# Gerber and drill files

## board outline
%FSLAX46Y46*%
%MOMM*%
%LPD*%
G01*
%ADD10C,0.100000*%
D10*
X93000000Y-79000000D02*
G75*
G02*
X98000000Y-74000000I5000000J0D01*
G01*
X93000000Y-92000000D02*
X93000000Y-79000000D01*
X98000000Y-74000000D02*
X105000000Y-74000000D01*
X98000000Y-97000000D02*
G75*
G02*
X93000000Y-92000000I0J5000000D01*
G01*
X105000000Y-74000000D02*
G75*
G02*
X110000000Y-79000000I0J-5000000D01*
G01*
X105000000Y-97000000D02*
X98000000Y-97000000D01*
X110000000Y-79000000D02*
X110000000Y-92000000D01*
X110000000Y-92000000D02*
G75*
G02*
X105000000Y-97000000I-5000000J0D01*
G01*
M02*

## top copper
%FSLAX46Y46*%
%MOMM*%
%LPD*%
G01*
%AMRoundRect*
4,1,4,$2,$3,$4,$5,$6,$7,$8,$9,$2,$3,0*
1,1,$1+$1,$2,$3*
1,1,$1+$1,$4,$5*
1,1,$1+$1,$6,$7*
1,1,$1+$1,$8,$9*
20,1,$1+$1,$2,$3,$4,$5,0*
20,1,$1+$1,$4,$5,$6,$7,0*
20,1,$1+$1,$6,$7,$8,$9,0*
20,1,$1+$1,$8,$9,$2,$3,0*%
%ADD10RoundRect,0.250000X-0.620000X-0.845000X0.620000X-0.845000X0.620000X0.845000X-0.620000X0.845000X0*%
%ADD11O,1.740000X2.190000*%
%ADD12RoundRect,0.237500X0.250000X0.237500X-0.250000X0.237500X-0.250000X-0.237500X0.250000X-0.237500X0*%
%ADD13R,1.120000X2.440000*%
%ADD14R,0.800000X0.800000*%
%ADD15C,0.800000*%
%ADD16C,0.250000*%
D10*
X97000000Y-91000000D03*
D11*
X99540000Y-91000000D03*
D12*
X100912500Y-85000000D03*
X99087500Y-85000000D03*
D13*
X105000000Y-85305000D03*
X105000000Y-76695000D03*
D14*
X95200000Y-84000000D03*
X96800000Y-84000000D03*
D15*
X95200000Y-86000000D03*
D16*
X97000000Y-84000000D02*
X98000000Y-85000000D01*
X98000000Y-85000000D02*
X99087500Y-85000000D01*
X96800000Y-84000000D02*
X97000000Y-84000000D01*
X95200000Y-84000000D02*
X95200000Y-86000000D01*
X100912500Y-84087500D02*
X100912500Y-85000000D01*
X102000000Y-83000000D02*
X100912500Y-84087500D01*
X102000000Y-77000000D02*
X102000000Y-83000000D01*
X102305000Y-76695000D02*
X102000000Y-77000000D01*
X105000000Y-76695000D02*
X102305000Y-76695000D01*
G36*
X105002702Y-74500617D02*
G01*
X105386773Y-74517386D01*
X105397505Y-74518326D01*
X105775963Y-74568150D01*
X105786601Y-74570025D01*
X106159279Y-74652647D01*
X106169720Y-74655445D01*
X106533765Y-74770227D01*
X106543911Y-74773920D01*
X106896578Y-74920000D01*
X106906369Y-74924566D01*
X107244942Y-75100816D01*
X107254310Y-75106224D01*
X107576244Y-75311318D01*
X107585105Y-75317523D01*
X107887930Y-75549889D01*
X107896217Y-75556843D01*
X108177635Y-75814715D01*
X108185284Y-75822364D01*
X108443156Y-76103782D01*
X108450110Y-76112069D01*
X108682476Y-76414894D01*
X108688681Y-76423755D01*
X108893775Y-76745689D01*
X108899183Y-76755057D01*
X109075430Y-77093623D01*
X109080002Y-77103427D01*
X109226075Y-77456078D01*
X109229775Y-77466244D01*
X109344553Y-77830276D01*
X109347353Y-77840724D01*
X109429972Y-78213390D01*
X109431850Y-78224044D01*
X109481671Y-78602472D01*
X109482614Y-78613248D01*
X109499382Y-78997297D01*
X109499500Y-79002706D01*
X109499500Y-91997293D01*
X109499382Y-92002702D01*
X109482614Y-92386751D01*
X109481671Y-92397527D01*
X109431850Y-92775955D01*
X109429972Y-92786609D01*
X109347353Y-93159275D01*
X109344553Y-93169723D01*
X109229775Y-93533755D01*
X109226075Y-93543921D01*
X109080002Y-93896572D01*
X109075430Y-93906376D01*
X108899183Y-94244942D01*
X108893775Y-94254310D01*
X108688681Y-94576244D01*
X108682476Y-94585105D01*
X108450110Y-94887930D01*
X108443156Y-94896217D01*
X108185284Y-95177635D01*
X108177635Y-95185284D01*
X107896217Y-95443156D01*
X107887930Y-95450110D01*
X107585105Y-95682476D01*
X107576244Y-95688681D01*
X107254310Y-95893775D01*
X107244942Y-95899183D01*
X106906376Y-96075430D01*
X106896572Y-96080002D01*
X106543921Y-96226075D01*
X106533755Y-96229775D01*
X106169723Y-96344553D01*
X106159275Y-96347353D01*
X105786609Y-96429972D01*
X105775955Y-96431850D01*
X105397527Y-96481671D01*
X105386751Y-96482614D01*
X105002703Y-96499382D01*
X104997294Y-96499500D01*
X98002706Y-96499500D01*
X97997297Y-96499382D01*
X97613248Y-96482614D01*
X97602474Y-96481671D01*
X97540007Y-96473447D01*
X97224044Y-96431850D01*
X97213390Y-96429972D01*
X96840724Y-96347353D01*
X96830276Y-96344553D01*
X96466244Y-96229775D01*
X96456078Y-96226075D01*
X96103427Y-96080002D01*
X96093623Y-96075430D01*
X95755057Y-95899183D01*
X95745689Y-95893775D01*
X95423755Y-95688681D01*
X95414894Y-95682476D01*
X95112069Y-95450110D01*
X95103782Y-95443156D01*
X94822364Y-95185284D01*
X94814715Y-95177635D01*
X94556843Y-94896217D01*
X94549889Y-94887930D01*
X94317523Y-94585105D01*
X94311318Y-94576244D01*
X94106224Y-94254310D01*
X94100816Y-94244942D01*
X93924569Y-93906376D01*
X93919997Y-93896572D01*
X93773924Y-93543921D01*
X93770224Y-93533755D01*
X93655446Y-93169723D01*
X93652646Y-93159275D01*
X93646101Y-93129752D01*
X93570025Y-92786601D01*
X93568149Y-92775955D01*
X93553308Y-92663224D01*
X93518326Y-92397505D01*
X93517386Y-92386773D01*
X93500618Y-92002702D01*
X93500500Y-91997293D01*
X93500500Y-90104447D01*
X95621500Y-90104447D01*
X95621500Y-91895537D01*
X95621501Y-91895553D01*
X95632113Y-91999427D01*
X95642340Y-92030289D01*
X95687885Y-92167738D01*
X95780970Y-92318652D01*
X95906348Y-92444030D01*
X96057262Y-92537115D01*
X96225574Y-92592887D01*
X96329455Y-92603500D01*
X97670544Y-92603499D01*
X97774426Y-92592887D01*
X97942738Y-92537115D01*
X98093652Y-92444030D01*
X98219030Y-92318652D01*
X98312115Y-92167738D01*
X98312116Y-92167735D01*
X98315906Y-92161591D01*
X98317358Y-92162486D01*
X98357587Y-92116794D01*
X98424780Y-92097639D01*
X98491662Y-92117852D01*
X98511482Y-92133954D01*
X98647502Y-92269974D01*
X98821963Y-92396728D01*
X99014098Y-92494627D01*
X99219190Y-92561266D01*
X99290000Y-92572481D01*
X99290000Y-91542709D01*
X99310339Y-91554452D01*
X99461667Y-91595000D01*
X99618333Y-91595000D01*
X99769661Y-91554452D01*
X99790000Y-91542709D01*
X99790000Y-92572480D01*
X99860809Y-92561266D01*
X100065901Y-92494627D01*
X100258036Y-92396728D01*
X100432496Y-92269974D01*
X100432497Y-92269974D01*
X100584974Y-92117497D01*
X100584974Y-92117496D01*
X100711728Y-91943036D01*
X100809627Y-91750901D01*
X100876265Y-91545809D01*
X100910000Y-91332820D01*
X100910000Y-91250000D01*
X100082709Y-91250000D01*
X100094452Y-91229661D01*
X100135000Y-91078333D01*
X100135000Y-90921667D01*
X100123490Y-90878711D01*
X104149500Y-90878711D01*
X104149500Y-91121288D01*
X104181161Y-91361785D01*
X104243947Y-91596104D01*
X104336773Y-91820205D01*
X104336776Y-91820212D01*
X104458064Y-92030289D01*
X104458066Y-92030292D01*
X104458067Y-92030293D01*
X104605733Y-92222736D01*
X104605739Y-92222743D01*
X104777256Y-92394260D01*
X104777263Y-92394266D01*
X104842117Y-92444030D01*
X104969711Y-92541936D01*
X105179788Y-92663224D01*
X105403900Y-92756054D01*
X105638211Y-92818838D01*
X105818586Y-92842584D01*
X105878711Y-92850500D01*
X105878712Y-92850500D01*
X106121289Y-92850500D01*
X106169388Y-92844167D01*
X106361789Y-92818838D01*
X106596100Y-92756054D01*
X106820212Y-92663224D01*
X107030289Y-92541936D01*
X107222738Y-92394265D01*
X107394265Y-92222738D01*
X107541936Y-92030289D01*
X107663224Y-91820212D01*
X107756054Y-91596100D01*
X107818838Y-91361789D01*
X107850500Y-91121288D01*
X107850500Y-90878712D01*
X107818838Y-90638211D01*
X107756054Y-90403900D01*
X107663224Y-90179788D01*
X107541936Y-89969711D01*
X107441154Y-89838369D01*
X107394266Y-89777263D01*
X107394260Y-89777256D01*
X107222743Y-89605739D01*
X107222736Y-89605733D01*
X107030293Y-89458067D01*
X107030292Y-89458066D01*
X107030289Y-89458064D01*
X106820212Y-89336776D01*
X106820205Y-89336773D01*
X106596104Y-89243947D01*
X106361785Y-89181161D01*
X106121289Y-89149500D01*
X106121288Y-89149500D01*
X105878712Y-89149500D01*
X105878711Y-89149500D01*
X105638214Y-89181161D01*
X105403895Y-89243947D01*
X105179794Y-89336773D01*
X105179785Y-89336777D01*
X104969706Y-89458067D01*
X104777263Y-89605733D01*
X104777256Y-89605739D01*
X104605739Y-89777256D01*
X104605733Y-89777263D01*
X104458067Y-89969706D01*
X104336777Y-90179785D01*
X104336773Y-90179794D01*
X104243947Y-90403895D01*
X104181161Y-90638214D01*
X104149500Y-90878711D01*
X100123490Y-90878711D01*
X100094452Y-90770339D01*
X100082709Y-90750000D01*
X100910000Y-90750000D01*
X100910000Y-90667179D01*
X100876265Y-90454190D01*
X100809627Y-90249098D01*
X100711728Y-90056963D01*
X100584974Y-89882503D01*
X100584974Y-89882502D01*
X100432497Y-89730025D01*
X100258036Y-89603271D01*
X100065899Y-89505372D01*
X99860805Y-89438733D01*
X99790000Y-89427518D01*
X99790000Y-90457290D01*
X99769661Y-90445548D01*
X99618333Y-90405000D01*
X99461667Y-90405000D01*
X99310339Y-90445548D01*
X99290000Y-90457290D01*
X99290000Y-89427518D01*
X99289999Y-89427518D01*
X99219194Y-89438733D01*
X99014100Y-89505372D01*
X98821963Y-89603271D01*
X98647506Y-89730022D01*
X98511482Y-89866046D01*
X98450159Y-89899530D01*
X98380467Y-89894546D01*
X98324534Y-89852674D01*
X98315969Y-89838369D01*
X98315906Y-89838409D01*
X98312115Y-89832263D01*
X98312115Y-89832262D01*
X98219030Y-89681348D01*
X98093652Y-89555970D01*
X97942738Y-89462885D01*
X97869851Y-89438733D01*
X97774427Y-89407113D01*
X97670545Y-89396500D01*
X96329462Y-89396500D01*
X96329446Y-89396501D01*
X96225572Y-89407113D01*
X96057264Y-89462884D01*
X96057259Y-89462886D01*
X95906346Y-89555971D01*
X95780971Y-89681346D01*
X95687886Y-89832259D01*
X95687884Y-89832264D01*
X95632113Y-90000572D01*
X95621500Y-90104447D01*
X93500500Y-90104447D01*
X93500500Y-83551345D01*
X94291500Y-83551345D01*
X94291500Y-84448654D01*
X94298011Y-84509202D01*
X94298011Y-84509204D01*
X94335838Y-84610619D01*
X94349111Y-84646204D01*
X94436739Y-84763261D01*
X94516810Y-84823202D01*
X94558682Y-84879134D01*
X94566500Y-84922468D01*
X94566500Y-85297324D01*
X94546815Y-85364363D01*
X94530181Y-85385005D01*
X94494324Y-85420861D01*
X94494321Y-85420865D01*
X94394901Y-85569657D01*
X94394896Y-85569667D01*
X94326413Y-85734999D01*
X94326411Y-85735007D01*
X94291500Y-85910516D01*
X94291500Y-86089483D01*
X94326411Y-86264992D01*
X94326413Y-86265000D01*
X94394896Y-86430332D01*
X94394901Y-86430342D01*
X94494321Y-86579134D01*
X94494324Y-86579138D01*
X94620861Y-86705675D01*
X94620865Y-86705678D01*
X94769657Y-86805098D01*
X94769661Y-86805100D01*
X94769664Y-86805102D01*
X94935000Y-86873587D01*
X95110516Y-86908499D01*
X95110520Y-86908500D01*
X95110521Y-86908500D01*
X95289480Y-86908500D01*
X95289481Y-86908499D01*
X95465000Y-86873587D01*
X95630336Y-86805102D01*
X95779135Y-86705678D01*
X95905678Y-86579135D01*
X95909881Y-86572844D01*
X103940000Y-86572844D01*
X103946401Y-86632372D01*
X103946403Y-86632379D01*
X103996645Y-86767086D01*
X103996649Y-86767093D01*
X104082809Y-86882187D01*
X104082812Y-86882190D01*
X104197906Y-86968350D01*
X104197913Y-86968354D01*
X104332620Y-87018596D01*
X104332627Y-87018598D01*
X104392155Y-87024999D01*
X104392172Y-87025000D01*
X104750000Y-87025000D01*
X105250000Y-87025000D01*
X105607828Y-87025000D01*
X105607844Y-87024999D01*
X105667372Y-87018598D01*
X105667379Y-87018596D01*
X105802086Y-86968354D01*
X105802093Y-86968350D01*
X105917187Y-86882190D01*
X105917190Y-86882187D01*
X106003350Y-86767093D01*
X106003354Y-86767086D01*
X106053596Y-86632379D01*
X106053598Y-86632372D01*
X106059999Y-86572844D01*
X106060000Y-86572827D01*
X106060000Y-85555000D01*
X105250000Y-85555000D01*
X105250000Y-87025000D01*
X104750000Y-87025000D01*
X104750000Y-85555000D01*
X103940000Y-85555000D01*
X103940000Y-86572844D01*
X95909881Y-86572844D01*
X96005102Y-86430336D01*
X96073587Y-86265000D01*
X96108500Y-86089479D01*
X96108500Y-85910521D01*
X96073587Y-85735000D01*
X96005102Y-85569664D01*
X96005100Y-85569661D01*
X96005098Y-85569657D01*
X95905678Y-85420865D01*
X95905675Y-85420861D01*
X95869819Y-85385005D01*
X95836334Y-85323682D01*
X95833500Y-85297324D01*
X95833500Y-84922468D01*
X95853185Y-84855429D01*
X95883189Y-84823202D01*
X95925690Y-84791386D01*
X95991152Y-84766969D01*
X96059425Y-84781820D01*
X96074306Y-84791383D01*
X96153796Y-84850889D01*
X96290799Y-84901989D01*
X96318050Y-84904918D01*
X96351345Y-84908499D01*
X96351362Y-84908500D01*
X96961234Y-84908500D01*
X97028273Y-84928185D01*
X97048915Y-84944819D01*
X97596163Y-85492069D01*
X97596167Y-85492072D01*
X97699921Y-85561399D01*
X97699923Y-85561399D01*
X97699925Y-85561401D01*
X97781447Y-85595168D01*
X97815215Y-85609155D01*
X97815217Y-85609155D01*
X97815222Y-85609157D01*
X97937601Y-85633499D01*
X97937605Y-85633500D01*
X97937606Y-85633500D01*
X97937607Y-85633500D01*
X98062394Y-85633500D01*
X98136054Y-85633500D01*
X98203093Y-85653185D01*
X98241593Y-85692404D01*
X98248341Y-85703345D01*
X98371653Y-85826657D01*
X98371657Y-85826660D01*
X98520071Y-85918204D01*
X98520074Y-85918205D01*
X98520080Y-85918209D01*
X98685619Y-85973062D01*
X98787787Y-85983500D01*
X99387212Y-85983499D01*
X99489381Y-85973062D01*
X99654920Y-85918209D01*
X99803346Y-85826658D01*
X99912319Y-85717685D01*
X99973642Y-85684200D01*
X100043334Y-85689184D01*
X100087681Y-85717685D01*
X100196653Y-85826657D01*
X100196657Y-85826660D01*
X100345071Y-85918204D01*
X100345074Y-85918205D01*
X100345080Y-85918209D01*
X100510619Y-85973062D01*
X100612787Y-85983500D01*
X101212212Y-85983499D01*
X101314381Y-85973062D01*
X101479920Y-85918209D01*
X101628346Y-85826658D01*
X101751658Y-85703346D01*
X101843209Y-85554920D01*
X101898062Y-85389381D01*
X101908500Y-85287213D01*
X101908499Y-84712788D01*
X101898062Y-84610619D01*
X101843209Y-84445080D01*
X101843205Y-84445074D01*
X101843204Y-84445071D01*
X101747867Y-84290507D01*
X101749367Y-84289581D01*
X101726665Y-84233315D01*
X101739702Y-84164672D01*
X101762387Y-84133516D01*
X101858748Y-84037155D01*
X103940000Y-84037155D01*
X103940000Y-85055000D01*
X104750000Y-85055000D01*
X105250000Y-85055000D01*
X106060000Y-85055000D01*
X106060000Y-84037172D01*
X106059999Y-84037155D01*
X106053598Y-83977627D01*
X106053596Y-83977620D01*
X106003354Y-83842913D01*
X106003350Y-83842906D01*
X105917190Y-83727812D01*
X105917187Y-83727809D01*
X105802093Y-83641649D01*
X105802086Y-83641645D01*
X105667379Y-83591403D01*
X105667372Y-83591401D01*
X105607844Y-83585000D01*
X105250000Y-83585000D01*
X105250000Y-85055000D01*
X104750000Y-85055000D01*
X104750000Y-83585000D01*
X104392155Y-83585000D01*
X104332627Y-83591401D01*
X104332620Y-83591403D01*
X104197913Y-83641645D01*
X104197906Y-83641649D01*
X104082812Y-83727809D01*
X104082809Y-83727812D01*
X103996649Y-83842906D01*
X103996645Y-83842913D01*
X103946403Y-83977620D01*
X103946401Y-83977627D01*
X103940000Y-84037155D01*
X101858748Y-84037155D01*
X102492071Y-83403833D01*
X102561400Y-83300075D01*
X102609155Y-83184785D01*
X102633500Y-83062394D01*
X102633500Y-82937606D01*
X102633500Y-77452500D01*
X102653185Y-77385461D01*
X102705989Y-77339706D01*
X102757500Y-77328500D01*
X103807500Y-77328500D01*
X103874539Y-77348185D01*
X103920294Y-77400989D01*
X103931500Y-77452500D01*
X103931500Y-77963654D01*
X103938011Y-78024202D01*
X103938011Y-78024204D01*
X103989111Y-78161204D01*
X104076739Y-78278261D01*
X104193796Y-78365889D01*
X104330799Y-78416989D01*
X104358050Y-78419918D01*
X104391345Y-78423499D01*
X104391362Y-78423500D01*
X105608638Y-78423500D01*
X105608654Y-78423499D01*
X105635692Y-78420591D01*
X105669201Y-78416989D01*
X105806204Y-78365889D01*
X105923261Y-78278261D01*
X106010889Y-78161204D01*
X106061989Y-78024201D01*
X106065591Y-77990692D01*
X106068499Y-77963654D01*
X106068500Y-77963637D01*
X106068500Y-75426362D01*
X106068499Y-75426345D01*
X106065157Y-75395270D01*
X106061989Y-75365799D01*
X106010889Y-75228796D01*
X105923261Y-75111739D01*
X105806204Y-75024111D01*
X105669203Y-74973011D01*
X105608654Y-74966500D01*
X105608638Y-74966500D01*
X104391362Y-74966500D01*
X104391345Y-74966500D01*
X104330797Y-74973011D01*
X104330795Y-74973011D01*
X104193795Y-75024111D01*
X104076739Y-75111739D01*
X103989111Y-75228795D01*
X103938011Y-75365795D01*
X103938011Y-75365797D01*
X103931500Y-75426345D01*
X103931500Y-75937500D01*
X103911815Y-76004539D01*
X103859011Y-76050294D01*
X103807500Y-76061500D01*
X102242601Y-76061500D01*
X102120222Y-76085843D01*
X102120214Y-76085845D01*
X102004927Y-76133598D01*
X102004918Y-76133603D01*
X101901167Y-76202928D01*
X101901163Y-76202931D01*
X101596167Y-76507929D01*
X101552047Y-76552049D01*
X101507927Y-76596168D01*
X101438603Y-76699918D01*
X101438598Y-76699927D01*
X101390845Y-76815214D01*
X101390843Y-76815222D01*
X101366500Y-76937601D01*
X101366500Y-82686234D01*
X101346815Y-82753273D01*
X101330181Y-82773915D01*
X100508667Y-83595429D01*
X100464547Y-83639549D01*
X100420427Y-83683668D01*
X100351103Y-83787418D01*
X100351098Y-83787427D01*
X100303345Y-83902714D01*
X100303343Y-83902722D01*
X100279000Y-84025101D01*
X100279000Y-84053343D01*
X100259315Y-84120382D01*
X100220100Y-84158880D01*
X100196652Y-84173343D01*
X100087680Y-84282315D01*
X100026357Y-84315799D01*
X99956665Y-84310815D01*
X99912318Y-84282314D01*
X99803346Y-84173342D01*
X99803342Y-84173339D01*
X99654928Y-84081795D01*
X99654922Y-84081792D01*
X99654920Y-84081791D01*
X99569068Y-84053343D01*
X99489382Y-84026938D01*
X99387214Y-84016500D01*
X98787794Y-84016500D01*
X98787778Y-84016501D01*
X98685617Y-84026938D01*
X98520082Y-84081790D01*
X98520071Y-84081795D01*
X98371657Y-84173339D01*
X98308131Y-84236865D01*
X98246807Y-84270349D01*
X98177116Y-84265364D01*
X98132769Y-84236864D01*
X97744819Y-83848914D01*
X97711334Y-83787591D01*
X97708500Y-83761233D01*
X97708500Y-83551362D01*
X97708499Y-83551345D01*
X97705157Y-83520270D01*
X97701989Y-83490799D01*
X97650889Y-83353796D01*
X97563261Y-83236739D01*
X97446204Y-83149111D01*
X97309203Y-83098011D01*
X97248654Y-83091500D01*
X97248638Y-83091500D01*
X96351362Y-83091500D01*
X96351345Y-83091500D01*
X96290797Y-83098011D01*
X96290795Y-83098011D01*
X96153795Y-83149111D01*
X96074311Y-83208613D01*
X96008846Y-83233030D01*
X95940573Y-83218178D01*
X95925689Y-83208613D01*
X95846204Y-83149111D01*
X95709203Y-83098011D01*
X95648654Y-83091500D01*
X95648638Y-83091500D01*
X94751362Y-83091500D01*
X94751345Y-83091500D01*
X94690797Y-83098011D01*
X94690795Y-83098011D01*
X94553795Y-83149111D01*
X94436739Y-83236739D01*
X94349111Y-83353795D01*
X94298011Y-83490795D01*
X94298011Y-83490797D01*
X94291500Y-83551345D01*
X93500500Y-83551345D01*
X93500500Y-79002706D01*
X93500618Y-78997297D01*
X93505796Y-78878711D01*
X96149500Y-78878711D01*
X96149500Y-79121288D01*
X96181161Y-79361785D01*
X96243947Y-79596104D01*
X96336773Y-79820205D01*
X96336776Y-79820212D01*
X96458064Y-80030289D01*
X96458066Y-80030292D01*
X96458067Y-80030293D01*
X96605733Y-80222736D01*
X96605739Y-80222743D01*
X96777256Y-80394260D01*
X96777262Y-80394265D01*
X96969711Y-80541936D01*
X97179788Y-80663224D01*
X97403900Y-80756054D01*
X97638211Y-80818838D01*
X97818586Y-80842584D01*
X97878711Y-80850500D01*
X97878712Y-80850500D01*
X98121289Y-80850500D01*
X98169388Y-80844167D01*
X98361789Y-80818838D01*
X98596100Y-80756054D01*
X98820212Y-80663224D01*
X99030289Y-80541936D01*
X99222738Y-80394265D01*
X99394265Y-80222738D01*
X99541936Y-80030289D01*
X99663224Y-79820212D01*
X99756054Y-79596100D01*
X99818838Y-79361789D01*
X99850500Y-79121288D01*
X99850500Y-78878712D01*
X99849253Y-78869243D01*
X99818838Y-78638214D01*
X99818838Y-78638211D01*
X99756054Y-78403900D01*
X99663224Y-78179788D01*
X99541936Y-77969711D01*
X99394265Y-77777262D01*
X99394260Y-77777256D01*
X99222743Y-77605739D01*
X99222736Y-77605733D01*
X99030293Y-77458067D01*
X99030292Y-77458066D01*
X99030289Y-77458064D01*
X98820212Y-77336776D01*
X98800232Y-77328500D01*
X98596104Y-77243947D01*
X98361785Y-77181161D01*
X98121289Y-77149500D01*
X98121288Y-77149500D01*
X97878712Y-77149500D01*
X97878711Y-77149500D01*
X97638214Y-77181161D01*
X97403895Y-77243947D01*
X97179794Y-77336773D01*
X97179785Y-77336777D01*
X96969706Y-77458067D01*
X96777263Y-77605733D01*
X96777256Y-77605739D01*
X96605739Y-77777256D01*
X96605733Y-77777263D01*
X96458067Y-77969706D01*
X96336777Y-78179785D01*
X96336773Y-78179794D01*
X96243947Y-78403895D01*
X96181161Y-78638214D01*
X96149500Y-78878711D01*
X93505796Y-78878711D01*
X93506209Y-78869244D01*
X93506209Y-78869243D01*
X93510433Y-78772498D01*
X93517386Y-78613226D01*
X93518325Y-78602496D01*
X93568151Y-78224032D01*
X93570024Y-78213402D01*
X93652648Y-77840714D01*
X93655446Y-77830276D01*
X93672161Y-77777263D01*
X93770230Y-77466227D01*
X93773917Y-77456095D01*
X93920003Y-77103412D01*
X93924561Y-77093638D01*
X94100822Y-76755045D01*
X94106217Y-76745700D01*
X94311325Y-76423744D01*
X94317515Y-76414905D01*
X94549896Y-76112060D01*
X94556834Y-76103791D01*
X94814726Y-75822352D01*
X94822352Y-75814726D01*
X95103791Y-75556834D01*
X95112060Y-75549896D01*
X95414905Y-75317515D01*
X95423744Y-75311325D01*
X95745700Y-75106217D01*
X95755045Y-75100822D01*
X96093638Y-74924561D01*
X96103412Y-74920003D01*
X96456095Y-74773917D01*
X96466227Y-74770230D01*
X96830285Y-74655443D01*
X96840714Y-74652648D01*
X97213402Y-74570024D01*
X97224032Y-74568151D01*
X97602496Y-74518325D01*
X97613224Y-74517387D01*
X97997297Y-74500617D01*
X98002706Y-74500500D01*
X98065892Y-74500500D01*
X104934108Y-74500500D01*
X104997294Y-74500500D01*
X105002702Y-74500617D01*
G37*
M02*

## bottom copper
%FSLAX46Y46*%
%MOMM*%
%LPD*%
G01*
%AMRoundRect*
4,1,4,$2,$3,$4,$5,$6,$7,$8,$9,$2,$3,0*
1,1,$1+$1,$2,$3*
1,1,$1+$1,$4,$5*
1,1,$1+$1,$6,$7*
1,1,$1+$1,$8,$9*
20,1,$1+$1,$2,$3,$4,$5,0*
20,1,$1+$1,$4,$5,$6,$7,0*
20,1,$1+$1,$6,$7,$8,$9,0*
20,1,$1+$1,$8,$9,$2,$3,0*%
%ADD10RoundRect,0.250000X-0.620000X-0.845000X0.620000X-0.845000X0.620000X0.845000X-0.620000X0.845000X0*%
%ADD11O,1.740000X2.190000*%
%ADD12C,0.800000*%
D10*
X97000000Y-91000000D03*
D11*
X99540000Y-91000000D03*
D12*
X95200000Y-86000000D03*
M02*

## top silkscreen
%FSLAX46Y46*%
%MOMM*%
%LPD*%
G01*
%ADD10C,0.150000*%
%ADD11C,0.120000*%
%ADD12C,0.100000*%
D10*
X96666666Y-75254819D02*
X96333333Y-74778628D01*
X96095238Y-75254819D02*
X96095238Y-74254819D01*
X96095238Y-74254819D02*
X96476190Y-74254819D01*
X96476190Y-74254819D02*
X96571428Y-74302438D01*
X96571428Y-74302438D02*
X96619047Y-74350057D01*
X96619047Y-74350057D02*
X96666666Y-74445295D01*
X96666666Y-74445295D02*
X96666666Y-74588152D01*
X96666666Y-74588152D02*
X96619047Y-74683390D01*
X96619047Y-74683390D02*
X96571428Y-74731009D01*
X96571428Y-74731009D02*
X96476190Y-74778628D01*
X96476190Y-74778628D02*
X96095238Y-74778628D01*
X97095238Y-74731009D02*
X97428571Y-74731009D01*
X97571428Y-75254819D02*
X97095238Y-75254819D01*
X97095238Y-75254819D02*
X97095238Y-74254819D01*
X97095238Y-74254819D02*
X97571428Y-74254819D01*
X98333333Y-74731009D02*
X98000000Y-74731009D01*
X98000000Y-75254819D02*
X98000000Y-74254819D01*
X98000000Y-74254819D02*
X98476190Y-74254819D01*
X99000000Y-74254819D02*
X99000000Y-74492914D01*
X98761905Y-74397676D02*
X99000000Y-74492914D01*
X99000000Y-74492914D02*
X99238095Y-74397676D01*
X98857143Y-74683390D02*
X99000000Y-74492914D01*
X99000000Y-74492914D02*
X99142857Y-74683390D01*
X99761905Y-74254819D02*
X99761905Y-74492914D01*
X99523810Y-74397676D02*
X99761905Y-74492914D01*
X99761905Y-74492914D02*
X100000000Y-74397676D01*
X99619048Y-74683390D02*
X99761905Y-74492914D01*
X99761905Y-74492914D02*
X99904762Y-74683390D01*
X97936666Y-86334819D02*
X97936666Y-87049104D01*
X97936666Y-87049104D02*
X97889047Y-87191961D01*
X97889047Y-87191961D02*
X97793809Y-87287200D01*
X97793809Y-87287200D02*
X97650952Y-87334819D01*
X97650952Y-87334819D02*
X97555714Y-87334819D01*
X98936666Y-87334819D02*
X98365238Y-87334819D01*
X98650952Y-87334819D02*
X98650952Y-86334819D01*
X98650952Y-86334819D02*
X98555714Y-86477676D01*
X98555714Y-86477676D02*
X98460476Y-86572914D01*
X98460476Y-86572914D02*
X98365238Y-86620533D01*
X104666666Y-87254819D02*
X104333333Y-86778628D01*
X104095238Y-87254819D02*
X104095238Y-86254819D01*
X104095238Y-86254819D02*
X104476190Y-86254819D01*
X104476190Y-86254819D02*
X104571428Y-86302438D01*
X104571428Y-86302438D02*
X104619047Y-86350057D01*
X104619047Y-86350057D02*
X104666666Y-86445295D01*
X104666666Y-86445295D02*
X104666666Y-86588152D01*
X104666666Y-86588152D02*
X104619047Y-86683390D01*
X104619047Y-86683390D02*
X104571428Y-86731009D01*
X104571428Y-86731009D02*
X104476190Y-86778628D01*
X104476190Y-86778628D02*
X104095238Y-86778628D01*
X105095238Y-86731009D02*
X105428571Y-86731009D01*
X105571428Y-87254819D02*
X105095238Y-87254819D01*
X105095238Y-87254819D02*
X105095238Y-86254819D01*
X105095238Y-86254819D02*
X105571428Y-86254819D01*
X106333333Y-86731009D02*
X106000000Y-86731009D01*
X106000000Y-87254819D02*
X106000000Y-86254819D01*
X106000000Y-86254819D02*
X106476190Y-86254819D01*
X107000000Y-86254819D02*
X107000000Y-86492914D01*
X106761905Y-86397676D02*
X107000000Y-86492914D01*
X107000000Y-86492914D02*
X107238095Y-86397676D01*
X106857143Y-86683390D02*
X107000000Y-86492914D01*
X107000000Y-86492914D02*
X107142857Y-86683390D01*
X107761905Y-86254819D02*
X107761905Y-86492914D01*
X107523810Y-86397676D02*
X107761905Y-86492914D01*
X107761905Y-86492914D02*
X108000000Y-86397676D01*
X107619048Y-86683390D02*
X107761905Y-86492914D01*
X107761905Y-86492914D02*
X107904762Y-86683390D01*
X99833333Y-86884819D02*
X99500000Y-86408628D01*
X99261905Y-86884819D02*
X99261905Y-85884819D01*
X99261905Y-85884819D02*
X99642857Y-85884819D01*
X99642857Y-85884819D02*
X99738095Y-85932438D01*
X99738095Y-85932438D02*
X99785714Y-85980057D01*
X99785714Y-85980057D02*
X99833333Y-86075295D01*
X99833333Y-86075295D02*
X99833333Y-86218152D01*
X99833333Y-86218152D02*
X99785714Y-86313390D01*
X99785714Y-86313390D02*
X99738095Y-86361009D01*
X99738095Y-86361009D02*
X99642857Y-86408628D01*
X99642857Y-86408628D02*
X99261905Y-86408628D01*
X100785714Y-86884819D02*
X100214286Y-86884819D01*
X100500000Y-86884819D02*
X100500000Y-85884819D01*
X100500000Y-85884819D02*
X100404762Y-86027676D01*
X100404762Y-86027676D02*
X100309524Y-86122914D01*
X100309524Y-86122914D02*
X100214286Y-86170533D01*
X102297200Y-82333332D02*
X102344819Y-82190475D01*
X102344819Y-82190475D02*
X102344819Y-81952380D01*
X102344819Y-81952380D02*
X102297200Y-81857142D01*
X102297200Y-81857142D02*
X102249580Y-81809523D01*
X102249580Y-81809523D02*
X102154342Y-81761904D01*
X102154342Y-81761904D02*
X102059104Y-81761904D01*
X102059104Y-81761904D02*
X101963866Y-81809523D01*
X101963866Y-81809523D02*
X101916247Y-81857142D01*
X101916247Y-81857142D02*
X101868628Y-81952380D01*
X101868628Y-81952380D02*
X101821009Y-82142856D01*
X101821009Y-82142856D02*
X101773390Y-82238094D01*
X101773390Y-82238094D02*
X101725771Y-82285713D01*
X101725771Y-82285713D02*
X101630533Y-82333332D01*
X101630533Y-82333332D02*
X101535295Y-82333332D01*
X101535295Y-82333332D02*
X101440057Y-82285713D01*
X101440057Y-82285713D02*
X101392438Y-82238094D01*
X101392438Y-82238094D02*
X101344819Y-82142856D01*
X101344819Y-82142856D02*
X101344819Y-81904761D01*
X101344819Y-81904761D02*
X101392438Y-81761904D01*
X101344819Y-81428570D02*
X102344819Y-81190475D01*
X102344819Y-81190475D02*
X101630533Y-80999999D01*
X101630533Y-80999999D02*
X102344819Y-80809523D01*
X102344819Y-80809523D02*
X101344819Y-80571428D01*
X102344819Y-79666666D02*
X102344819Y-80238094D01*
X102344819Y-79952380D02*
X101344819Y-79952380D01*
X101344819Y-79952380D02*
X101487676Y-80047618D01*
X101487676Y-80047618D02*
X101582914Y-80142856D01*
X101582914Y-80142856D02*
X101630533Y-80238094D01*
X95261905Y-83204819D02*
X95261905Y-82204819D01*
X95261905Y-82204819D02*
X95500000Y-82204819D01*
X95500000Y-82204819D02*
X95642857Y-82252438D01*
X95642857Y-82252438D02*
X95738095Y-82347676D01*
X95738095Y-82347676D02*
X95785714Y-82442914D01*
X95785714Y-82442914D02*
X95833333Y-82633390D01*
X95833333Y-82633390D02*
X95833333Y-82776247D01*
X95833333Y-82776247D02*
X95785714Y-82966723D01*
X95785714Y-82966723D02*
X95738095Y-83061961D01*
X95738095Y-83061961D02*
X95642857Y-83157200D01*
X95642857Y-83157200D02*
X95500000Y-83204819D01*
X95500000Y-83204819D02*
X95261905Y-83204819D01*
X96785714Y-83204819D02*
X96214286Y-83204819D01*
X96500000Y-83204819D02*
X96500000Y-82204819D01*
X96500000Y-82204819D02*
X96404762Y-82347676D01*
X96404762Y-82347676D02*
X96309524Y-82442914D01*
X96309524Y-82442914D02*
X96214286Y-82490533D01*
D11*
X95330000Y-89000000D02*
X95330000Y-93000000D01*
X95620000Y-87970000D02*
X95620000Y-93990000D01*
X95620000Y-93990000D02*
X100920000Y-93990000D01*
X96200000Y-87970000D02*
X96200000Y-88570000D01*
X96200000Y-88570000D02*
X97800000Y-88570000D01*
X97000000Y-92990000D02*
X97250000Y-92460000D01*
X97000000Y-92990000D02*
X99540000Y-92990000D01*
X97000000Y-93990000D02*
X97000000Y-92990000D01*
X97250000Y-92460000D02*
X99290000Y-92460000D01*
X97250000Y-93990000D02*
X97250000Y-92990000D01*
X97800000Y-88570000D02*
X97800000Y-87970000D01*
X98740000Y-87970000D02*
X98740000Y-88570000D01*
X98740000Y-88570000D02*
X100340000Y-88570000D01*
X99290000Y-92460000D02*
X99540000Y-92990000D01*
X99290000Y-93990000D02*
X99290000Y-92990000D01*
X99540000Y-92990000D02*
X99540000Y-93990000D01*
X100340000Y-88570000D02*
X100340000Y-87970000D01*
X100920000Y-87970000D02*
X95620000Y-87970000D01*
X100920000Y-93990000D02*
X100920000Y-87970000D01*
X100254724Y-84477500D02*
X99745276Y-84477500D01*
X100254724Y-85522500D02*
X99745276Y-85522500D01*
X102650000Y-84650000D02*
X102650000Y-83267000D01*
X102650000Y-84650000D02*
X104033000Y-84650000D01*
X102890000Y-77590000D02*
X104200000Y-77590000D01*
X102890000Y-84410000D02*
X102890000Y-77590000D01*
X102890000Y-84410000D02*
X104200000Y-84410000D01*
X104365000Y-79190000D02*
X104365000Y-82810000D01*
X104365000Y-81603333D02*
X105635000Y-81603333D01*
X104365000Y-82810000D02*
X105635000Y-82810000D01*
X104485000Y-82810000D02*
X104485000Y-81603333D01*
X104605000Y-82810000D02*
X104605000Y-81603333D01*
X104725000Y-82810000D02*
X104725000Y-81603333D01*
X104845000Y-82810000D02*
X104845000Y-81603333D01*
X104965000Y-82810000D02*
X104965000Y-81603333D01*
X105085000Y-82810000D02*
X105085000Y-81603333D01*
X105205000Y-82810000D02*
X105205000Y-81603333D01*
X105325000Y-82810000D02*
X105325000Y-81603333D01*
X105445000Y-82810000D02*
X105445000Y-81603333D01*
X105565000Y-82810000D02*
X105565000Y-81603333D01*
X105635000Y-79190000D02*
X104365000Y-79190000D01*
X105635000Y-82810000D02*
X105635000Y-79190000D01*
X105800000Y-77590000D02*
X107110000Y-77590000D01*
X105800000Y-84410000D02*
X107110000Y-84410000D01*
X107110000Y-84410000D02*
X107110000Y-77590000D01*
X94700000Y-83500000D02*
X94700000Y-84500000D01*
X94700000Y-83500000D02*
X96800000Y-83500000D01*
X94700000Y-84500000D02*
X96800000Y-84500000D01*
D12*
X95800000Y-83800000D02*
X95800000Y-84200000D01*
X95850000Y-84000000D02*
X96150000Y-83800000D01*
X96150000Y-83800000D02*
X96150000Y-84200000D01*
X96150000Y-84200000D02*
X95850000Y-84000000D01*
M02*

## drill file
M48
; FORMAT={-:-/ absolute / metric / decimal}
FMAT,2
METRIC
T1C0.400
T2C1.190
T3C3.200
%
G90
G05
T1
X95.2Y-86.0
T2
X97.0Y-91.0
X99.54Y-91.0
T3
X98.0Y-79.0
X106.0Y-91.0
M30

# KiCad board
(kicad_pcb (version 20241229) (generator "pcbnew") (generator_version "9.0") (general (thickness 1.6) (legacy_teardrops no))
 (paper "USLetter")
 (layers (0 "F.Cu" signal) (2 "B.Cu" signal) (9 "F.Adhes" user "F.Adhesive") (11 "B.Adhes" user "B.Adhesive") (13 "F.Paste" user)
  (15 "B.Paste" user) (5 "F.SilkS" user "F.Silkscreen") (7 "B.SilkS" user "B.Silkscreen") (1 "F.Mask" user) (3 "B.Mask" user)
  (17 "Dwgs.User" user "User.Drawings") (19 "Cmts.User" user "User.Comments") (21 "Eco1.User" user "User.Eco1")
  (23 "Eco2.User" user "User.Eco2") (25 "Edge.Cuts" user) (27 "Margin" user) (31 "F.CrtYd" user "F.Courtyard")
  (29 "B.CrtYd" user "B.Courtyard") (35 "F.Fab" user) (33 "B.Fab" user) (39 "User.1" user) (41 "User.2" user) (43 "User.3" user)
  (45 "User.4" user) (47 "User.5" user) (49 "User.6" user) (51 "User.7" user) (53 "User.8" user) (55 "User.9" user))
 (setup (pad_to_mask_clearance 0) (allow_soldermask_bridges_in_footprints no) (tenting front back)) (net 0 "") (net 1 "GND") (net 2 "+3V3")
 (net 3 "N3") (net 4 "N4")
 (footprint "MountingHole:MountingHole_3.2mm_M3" (layer "F.Cu") (at 98 79)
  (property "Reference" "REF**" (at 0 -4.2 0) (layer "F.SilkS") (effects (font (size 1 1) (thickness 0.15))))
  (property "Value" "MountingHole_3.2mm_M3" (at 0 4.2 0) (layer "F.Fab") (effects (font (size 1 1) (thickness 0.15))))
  (pad "" np_thru_hole circle (at 0 0) (size 3.2 3.2) (drill 3.2) (layers "*.Cu" "*.Mask")))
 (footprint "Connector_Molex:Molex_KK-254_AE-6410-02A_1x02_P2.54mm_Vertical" (layer "F.Cu") (at 97 91)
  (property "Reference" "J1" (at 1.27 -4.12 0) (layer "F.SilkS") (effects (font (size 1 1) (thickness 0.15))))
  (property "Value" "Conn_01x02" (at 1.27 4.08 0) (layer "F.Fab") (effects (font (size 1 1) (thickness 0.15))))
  (fp_line (start -1.67 -2) (end -1.67 2) (stroke (width 0.12) (type solid)) (layer "F.SilkS"))
  (fp_line (start -1.38 -3.03) (end -1.38 2.99) (stroke (width 0.12) (type solid)) (layer "F.SilkS"))
  (fp_line (start -1.38 2.99) (end 3.92 2.99) (stroke (width 0.12) (type solid)) (layer "F.SilkS"))
  (fp_line (start -0.8 -3.03) (end -0.8 -2.43) (stroke (width 0.12) (type solid)) (layer "F.SilkS"))
  (fp_line (start -0.8 -2.43) (end 0.8 -2.43) (stroke (width 0.12) (type solid)) (layer "F.SilkS"))
  (fp_line (start 0 1.99) (end 0.25 1.46) (stroke (width 0.12) (type solid)) (layer "F.SilkS"))
  (fp_line (start 0 1.99) (end 2.54 1.99) (stroke (width 0.12) (type solid)) (layer "F.SilkS"))
  (fp_line (start 0 2.99) (end 0 1.99) (stroke (width 0.12) (type solid)) (layer "F.SilkS"))
  (fp_line (start 0.25 1.46) (end 2.29 1.46) (stroke (width 0.12) (type solid)) (layer "F.SilkS"))
  (fp_line (start 0.25 2.99) (end 0.25 1.99) (stroke (width 0.12) (type solid)) (layer "F.SilkS"))
  (fp_line (start 0.8 -2.43) (end 0.8 -3.03) (stroke (width 0.12) (type solid)) (layer "F.SilkS"))
  (fp_line (start 1.74 -3.03) (end 1.74 -2.43) (stroke (width 0.12) (type solid)) (layer "F.SilkS"))
  (fp_line (start 1.74 -2.43) (end 3.34 -2.43) (stroke (width 0.12) (type solid)) (layer "F.SilkS"))
  (fp_line (start 2.29 1.46) (end 2.54 1.99) (stroke (width 0.12) (type solid)) (layer "F.SilkS"))
  (fp_line (start 2.29 2.99) (end 2.29 1.99) (stroke (width 0.12) (type solid)) (layer "F.SilkS"))
  (fp_line (start 2.54 1.99) (end 2.54 2.99) (stroke (width 0.12) (type solid)) (layer "F.SilkS"))
  (fp_line (start 3.34 -2.43) (end 3.34 -3.03) (stroke (width 0.12) (type solid)) (layer "F.SilkS"))
  (fp_line (start 3.92 -3.03) (end -1.38 -3.03) (stroke (width 0.12) (type solid)) (layer "F.SilkS"))
  (fp_line (start 3.92 2.99) (end 3.92 -3.03) (stroke (width 0.12) (type solid)) (layer "F.SilkS"))
  (pad "1" thru_hole roundrect (at 0 0) (size 1.74 2.19) (drill 1.19) (layers "*.Cu" "*.Mask") (remove_unused_layers no)
   (roundrect_rratio 0.143678) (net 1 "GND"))
  (pad "2" thru_hole oval (at 2.54 0) (size 1.74 2.19) (drill 1.19) (layers "*.Cu" "*.Mask") (remove_unused_layers no) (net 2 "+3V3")))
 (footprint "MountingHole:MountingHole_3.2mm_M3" (layer "F.Cu") (at 106 91)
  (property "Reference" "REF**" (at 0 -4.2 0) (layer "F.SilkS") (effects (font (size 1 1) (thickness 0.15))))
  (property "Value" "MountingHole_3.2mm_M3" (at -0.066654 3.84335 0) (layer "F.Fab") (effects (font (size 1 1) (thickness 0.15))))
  (pad "" np_thru_hole circle (at 0 0) (size 3.2 3.2) (drill 3.2) (layers "*.Cu" "*.Mask")))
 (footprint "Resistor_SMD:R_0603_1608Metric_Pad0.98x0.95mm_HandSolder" (layer "F.Cu") (at 100 85 180)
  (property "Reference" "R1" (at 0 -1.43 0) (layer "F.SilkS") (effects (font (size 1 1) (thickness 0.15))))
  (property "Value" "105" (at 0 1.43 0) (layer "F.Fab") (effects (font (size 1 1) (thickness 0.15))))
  (fp_line (start -0.254724 0.5225) (end 0.254724 0.5225) (stroke (width 0.12) (type solid)) (layer "F.SilkS"))
  (fp_line (start -0.254724 -0.5225) (end 0.254724 -0.5225) (stroke (width 0.12) (type solid)) (layer "F.SilkS"))
  (pad "1" smd roundrect (at -0.9125 0 180) (size 0.975 0.95) (layers "F.Cu" "F.Mask" "F.Paste") (roundrect_rratio 0.25) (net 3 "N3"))
  (pad "2" smd roundrect (at 0.9125 0 180) (size 0.975 0.95) (layers "F.Cu" "F.Mask" "F.Paste") (roundrect_rratio 0.25) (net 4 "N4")))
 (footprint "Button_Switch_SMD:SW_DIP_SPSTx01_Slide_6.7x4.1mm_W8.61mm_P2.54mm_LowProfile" (layer "F.Cu") (at 105 81 90)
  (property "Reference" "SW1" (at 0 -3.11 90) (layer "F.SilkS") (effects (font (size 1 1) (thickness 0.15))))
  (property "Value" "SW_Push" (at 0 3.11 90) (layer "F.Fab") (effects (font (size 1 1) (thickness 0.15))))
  (fp_line (start -3.65 -2.35) (end -2.267 -2.35) (stroke (width 0.12) (type solid)) (layer "F.SilkS"))
  (fp_line (start -3.65 -2.35) (end -3.65 -0.967) (stroke (width 0.12) (type solid)) (layer "F.SilkS"))
  (fp_line (start 3.41 -2.11) (end 3.41 -0.8) (stroke (width 0.12) (type solid)) (layer "F.SilkS"))
  (fp_line (start -3.41 -2.11) (end 3.41 -2.11) (stroke (width 0.12) (type solid)) (layer "F.SilkS"))
  (fp_line (start -3.41 -2.11) (end -3.41 -0.8) (stroke (width 0.12) (type solid)) (layer "F.SilkS"))
  (fp_line (start 1.81 -0.635) (end -1.81 -0.635) (stroke (width 0.12) (type solid)) (layer "F.SilkS"))
  (fp_line (start -0.603333 -0.635) (end -0.603333 0.635) (stroke (width 0.12) (type solid)) (layer "F.SilkS"))
  (fp_line (start -1.81 -0.635) (end -1.81 0.635) (stroke (width 0.12) (type solid)) (layer "F.SilkS"))
  (fp_line (start -1.81 -0.515) (end -0.603333 -0.515) (stroke (width 0.12) (type solid)) (layer "F.SilkS"))
  (fp_line (start -1.81 -0.395) (end -0.603333 -0.395) (stroke (width 0.12) (type solid)) (layer "F.SilkS"))
  (fp_line (start -1.81 -0.275) (end -0.603333 -0.275) (stroke (width 0.12) (type solid)) (layer "F.SilkS"))
  (fp_line (start -1.81 -0.155) (end -0.603333 -0.155) (stroke (width 0.12) (type solid)) (layer "F.SilkS"))
  (fp_line (start -1.81 -0.035) (end -0.603333 -0.035) (stroke (width 0.12) (type solid)) (layer "F.SilkS"))
  (fp_line (start -1.81 0.085) (end -0.603333 0.085) (stroke (width 0.12) (type solid)) (layer "F.SilkS"))
  (fp_line (start -1.81 0.205) (end -0.603333 0.205) (stroke (width 0.12) (type solid)) (layer "F.SilkS"))
  (fp_line (start -1.81 0.325) (end -0.603333 0.325) (stroke (width 0.12) (type solid)) (layer "F.SilkS"))
  (fp_line (start -1.81 0.445) (end -0.603333 0.445) (stroke (width 0.12) (type solid)) (layer "F.SilkS"))
  (fp_line (start -1.81 0.565) (end -0.603333 0.565) (stroke (width 0.12) (type solid)) (layer "F.SilkS"))
  (fp_line (start 1.81 0.635) (end 1.81 -0.635) (stroke (width 0.12) (type solid)) (layer "F.SilkS"))
  (fp_line (start -1.81 0.635) (end 1.81 0.635) (stroke (width 0.12) (type solid)) (layer "F.SilkS"))
  (fp_line (start 3.41 0.8) (end 3.41 2.11) (stroke (width 0.12) (type solid)) (layer "F.SilkS"))
  (fp_line (start -3.41 0.8) (end -3.41 2.11) (stroke (width 0.12) (type solid)) (layer "F.SilkS"))
  (fp_line (start -3.41 2.11) (end 3.41 2.11) (stroke (width 0.12) (type solid)) (layer "F.SilkS"))
  (pad "1" smd rect (at -4.305 0 90) (size 2.44 1.12) (layers "F.Cu" "F.Mask" "F.Paste") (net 2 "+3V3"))
  (pad "2" smd rect (at 4.305 0 90) (size 2.44 1.12) (layers "F.Cu" "F.Mask" "F.Paste") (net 3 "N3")))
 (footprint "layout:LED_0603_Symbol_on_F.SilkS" (layer "F.Cu") (at 96 84)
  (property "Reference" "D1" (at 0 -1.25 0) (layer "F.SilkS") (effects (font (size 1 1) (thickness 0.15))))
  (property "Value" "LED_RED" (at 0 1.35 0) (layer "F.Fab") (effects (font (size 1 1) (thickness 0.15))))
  (fp_line (start -1.3 -0.5) (end -1.3 0.5) (stroke (width 0.12) (type solid)) (layer "F.SilkS"))
  (fp_line (start -1.3 -0.5) (end 0.8 -0.5) (stroke (width 0.12) (type solid)) (layer "F.SilkS"))
  (fp_line (start -1.3 0.5) (end 0.8 0.5) (stroke (width 0.12) (type solid)) (layer "F.SilkS"))
  (fp_line (start -0.2 -0.2) (end -0.2 0.2) (stroke (width 0.1) (type solid)) (layer "F.SilkS"))
  (fp_line (start -0.15 0) (end 0.15 -0.2) (stroke (width 0.1) (type solid)) (layer "F.SilkS"))
  (fp_line (start 0.15 -0.2) (end 0.15 0.2) (stroke (width 0.1) (type solid)) (layer "F.SilkS"))
  (fp_line (start 0.15 0.2) (end -0.15 0) (stroke (width 0.1) (type solid)) (layer "F.SilkS"))
  (pad "1" smd rect (at -0.8 0 180) (size 0.8 0.8) (layers "F.Cu" "F.Mask" "F.Paste") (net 1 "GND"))
  (pad "2" smd rect (at 0.8 0 180) (size 0.8 0.8) (layers "F.Cu" "F.Mask" "F.Paste") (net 4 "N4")))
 (gr_arc (start 93 79) (mid 94.464466 75.464466) (end 98 74) (stroke (width 0.1) (type default)) (layer "Edge.Cuts"))
 (gr_line (start 93 92) (end 93 79) (stroke (width 0.1) (type default)) (layer "Edge.Cuts"))
 (gr_line (start 98 74) (end 105 74) (stroke (width 0.1) (type default)) (layer "Edge.Cuts"))
 (gr_arc (start 98 97) (mid 94.464466 95.535534) (end 93 92) (stroke (width 0.1) (type default)) (layer "Edge.Cuts"))
 (gr_arc (start 105 74) (mid 108.535534 75.464466) (end 110 79) (stroke (width 0.1) (type default)) (layer "Edge.Cuts"))
 (gr_line (start 105 97) (end 98 97) (stroke (width 0.1) (type default)) (layer "Edge.Cuts"))
 (gr_line (start 110 79) (end 110 92) (stroke (width 0.1) (type default)) (layer "Edge.Cuts"))
 (gr_arc (start 110 92) (mid 108.535534 95.535534) (end 105 97) (stroke (width 0.1) (type default)) (layer "Edge.Cuts"))
 (segment (start 97 84) (end 98 85) (width 0.25) (layer "F.Cu") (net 4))
 (segment (start 98 85) (end 99.0875 85) (width 0.25) (layer "F.Cu") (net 4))
 (segment (start 96.8 84) (end 97 84) (width 0.25) (layer "F.Cu") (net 4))
 (segment (start 95.2 84) (end 95.2 86) (width 0.25) (layer "F.Cu") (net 1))
 (via (at 95.2 86) (size 0.8) (drill 0.4) (layers "F.Cu" "B.Cu") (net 1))
 (segment (start 100.9125 84.0875) (end 100.9125 85) (width 0.25) (layer "F.Cu") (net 3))
 (segment (start 102 83) (end 100.9125 84.0875) (width 0.25) (layer "F.Cu") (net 3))
 (segment (start 102 77) (end 102 83) (width 0.25) (layer "F.Cu") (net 3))
 (segment (start 102.305 76.695) (end 102 77) (width 0.25) (layer "F.Cu") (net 3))
 (segment (start 105 76.695) (end 102.305 76.695) (width 0.25) (layer "F.Cu") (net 3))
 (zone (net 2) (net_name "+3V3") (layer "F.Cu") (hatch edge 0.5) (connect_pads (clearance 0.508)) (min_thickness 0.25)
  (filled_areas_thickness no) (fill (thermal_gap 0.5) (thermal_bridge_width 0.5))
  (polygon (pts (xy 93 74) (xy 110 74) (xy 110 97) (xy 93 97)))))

